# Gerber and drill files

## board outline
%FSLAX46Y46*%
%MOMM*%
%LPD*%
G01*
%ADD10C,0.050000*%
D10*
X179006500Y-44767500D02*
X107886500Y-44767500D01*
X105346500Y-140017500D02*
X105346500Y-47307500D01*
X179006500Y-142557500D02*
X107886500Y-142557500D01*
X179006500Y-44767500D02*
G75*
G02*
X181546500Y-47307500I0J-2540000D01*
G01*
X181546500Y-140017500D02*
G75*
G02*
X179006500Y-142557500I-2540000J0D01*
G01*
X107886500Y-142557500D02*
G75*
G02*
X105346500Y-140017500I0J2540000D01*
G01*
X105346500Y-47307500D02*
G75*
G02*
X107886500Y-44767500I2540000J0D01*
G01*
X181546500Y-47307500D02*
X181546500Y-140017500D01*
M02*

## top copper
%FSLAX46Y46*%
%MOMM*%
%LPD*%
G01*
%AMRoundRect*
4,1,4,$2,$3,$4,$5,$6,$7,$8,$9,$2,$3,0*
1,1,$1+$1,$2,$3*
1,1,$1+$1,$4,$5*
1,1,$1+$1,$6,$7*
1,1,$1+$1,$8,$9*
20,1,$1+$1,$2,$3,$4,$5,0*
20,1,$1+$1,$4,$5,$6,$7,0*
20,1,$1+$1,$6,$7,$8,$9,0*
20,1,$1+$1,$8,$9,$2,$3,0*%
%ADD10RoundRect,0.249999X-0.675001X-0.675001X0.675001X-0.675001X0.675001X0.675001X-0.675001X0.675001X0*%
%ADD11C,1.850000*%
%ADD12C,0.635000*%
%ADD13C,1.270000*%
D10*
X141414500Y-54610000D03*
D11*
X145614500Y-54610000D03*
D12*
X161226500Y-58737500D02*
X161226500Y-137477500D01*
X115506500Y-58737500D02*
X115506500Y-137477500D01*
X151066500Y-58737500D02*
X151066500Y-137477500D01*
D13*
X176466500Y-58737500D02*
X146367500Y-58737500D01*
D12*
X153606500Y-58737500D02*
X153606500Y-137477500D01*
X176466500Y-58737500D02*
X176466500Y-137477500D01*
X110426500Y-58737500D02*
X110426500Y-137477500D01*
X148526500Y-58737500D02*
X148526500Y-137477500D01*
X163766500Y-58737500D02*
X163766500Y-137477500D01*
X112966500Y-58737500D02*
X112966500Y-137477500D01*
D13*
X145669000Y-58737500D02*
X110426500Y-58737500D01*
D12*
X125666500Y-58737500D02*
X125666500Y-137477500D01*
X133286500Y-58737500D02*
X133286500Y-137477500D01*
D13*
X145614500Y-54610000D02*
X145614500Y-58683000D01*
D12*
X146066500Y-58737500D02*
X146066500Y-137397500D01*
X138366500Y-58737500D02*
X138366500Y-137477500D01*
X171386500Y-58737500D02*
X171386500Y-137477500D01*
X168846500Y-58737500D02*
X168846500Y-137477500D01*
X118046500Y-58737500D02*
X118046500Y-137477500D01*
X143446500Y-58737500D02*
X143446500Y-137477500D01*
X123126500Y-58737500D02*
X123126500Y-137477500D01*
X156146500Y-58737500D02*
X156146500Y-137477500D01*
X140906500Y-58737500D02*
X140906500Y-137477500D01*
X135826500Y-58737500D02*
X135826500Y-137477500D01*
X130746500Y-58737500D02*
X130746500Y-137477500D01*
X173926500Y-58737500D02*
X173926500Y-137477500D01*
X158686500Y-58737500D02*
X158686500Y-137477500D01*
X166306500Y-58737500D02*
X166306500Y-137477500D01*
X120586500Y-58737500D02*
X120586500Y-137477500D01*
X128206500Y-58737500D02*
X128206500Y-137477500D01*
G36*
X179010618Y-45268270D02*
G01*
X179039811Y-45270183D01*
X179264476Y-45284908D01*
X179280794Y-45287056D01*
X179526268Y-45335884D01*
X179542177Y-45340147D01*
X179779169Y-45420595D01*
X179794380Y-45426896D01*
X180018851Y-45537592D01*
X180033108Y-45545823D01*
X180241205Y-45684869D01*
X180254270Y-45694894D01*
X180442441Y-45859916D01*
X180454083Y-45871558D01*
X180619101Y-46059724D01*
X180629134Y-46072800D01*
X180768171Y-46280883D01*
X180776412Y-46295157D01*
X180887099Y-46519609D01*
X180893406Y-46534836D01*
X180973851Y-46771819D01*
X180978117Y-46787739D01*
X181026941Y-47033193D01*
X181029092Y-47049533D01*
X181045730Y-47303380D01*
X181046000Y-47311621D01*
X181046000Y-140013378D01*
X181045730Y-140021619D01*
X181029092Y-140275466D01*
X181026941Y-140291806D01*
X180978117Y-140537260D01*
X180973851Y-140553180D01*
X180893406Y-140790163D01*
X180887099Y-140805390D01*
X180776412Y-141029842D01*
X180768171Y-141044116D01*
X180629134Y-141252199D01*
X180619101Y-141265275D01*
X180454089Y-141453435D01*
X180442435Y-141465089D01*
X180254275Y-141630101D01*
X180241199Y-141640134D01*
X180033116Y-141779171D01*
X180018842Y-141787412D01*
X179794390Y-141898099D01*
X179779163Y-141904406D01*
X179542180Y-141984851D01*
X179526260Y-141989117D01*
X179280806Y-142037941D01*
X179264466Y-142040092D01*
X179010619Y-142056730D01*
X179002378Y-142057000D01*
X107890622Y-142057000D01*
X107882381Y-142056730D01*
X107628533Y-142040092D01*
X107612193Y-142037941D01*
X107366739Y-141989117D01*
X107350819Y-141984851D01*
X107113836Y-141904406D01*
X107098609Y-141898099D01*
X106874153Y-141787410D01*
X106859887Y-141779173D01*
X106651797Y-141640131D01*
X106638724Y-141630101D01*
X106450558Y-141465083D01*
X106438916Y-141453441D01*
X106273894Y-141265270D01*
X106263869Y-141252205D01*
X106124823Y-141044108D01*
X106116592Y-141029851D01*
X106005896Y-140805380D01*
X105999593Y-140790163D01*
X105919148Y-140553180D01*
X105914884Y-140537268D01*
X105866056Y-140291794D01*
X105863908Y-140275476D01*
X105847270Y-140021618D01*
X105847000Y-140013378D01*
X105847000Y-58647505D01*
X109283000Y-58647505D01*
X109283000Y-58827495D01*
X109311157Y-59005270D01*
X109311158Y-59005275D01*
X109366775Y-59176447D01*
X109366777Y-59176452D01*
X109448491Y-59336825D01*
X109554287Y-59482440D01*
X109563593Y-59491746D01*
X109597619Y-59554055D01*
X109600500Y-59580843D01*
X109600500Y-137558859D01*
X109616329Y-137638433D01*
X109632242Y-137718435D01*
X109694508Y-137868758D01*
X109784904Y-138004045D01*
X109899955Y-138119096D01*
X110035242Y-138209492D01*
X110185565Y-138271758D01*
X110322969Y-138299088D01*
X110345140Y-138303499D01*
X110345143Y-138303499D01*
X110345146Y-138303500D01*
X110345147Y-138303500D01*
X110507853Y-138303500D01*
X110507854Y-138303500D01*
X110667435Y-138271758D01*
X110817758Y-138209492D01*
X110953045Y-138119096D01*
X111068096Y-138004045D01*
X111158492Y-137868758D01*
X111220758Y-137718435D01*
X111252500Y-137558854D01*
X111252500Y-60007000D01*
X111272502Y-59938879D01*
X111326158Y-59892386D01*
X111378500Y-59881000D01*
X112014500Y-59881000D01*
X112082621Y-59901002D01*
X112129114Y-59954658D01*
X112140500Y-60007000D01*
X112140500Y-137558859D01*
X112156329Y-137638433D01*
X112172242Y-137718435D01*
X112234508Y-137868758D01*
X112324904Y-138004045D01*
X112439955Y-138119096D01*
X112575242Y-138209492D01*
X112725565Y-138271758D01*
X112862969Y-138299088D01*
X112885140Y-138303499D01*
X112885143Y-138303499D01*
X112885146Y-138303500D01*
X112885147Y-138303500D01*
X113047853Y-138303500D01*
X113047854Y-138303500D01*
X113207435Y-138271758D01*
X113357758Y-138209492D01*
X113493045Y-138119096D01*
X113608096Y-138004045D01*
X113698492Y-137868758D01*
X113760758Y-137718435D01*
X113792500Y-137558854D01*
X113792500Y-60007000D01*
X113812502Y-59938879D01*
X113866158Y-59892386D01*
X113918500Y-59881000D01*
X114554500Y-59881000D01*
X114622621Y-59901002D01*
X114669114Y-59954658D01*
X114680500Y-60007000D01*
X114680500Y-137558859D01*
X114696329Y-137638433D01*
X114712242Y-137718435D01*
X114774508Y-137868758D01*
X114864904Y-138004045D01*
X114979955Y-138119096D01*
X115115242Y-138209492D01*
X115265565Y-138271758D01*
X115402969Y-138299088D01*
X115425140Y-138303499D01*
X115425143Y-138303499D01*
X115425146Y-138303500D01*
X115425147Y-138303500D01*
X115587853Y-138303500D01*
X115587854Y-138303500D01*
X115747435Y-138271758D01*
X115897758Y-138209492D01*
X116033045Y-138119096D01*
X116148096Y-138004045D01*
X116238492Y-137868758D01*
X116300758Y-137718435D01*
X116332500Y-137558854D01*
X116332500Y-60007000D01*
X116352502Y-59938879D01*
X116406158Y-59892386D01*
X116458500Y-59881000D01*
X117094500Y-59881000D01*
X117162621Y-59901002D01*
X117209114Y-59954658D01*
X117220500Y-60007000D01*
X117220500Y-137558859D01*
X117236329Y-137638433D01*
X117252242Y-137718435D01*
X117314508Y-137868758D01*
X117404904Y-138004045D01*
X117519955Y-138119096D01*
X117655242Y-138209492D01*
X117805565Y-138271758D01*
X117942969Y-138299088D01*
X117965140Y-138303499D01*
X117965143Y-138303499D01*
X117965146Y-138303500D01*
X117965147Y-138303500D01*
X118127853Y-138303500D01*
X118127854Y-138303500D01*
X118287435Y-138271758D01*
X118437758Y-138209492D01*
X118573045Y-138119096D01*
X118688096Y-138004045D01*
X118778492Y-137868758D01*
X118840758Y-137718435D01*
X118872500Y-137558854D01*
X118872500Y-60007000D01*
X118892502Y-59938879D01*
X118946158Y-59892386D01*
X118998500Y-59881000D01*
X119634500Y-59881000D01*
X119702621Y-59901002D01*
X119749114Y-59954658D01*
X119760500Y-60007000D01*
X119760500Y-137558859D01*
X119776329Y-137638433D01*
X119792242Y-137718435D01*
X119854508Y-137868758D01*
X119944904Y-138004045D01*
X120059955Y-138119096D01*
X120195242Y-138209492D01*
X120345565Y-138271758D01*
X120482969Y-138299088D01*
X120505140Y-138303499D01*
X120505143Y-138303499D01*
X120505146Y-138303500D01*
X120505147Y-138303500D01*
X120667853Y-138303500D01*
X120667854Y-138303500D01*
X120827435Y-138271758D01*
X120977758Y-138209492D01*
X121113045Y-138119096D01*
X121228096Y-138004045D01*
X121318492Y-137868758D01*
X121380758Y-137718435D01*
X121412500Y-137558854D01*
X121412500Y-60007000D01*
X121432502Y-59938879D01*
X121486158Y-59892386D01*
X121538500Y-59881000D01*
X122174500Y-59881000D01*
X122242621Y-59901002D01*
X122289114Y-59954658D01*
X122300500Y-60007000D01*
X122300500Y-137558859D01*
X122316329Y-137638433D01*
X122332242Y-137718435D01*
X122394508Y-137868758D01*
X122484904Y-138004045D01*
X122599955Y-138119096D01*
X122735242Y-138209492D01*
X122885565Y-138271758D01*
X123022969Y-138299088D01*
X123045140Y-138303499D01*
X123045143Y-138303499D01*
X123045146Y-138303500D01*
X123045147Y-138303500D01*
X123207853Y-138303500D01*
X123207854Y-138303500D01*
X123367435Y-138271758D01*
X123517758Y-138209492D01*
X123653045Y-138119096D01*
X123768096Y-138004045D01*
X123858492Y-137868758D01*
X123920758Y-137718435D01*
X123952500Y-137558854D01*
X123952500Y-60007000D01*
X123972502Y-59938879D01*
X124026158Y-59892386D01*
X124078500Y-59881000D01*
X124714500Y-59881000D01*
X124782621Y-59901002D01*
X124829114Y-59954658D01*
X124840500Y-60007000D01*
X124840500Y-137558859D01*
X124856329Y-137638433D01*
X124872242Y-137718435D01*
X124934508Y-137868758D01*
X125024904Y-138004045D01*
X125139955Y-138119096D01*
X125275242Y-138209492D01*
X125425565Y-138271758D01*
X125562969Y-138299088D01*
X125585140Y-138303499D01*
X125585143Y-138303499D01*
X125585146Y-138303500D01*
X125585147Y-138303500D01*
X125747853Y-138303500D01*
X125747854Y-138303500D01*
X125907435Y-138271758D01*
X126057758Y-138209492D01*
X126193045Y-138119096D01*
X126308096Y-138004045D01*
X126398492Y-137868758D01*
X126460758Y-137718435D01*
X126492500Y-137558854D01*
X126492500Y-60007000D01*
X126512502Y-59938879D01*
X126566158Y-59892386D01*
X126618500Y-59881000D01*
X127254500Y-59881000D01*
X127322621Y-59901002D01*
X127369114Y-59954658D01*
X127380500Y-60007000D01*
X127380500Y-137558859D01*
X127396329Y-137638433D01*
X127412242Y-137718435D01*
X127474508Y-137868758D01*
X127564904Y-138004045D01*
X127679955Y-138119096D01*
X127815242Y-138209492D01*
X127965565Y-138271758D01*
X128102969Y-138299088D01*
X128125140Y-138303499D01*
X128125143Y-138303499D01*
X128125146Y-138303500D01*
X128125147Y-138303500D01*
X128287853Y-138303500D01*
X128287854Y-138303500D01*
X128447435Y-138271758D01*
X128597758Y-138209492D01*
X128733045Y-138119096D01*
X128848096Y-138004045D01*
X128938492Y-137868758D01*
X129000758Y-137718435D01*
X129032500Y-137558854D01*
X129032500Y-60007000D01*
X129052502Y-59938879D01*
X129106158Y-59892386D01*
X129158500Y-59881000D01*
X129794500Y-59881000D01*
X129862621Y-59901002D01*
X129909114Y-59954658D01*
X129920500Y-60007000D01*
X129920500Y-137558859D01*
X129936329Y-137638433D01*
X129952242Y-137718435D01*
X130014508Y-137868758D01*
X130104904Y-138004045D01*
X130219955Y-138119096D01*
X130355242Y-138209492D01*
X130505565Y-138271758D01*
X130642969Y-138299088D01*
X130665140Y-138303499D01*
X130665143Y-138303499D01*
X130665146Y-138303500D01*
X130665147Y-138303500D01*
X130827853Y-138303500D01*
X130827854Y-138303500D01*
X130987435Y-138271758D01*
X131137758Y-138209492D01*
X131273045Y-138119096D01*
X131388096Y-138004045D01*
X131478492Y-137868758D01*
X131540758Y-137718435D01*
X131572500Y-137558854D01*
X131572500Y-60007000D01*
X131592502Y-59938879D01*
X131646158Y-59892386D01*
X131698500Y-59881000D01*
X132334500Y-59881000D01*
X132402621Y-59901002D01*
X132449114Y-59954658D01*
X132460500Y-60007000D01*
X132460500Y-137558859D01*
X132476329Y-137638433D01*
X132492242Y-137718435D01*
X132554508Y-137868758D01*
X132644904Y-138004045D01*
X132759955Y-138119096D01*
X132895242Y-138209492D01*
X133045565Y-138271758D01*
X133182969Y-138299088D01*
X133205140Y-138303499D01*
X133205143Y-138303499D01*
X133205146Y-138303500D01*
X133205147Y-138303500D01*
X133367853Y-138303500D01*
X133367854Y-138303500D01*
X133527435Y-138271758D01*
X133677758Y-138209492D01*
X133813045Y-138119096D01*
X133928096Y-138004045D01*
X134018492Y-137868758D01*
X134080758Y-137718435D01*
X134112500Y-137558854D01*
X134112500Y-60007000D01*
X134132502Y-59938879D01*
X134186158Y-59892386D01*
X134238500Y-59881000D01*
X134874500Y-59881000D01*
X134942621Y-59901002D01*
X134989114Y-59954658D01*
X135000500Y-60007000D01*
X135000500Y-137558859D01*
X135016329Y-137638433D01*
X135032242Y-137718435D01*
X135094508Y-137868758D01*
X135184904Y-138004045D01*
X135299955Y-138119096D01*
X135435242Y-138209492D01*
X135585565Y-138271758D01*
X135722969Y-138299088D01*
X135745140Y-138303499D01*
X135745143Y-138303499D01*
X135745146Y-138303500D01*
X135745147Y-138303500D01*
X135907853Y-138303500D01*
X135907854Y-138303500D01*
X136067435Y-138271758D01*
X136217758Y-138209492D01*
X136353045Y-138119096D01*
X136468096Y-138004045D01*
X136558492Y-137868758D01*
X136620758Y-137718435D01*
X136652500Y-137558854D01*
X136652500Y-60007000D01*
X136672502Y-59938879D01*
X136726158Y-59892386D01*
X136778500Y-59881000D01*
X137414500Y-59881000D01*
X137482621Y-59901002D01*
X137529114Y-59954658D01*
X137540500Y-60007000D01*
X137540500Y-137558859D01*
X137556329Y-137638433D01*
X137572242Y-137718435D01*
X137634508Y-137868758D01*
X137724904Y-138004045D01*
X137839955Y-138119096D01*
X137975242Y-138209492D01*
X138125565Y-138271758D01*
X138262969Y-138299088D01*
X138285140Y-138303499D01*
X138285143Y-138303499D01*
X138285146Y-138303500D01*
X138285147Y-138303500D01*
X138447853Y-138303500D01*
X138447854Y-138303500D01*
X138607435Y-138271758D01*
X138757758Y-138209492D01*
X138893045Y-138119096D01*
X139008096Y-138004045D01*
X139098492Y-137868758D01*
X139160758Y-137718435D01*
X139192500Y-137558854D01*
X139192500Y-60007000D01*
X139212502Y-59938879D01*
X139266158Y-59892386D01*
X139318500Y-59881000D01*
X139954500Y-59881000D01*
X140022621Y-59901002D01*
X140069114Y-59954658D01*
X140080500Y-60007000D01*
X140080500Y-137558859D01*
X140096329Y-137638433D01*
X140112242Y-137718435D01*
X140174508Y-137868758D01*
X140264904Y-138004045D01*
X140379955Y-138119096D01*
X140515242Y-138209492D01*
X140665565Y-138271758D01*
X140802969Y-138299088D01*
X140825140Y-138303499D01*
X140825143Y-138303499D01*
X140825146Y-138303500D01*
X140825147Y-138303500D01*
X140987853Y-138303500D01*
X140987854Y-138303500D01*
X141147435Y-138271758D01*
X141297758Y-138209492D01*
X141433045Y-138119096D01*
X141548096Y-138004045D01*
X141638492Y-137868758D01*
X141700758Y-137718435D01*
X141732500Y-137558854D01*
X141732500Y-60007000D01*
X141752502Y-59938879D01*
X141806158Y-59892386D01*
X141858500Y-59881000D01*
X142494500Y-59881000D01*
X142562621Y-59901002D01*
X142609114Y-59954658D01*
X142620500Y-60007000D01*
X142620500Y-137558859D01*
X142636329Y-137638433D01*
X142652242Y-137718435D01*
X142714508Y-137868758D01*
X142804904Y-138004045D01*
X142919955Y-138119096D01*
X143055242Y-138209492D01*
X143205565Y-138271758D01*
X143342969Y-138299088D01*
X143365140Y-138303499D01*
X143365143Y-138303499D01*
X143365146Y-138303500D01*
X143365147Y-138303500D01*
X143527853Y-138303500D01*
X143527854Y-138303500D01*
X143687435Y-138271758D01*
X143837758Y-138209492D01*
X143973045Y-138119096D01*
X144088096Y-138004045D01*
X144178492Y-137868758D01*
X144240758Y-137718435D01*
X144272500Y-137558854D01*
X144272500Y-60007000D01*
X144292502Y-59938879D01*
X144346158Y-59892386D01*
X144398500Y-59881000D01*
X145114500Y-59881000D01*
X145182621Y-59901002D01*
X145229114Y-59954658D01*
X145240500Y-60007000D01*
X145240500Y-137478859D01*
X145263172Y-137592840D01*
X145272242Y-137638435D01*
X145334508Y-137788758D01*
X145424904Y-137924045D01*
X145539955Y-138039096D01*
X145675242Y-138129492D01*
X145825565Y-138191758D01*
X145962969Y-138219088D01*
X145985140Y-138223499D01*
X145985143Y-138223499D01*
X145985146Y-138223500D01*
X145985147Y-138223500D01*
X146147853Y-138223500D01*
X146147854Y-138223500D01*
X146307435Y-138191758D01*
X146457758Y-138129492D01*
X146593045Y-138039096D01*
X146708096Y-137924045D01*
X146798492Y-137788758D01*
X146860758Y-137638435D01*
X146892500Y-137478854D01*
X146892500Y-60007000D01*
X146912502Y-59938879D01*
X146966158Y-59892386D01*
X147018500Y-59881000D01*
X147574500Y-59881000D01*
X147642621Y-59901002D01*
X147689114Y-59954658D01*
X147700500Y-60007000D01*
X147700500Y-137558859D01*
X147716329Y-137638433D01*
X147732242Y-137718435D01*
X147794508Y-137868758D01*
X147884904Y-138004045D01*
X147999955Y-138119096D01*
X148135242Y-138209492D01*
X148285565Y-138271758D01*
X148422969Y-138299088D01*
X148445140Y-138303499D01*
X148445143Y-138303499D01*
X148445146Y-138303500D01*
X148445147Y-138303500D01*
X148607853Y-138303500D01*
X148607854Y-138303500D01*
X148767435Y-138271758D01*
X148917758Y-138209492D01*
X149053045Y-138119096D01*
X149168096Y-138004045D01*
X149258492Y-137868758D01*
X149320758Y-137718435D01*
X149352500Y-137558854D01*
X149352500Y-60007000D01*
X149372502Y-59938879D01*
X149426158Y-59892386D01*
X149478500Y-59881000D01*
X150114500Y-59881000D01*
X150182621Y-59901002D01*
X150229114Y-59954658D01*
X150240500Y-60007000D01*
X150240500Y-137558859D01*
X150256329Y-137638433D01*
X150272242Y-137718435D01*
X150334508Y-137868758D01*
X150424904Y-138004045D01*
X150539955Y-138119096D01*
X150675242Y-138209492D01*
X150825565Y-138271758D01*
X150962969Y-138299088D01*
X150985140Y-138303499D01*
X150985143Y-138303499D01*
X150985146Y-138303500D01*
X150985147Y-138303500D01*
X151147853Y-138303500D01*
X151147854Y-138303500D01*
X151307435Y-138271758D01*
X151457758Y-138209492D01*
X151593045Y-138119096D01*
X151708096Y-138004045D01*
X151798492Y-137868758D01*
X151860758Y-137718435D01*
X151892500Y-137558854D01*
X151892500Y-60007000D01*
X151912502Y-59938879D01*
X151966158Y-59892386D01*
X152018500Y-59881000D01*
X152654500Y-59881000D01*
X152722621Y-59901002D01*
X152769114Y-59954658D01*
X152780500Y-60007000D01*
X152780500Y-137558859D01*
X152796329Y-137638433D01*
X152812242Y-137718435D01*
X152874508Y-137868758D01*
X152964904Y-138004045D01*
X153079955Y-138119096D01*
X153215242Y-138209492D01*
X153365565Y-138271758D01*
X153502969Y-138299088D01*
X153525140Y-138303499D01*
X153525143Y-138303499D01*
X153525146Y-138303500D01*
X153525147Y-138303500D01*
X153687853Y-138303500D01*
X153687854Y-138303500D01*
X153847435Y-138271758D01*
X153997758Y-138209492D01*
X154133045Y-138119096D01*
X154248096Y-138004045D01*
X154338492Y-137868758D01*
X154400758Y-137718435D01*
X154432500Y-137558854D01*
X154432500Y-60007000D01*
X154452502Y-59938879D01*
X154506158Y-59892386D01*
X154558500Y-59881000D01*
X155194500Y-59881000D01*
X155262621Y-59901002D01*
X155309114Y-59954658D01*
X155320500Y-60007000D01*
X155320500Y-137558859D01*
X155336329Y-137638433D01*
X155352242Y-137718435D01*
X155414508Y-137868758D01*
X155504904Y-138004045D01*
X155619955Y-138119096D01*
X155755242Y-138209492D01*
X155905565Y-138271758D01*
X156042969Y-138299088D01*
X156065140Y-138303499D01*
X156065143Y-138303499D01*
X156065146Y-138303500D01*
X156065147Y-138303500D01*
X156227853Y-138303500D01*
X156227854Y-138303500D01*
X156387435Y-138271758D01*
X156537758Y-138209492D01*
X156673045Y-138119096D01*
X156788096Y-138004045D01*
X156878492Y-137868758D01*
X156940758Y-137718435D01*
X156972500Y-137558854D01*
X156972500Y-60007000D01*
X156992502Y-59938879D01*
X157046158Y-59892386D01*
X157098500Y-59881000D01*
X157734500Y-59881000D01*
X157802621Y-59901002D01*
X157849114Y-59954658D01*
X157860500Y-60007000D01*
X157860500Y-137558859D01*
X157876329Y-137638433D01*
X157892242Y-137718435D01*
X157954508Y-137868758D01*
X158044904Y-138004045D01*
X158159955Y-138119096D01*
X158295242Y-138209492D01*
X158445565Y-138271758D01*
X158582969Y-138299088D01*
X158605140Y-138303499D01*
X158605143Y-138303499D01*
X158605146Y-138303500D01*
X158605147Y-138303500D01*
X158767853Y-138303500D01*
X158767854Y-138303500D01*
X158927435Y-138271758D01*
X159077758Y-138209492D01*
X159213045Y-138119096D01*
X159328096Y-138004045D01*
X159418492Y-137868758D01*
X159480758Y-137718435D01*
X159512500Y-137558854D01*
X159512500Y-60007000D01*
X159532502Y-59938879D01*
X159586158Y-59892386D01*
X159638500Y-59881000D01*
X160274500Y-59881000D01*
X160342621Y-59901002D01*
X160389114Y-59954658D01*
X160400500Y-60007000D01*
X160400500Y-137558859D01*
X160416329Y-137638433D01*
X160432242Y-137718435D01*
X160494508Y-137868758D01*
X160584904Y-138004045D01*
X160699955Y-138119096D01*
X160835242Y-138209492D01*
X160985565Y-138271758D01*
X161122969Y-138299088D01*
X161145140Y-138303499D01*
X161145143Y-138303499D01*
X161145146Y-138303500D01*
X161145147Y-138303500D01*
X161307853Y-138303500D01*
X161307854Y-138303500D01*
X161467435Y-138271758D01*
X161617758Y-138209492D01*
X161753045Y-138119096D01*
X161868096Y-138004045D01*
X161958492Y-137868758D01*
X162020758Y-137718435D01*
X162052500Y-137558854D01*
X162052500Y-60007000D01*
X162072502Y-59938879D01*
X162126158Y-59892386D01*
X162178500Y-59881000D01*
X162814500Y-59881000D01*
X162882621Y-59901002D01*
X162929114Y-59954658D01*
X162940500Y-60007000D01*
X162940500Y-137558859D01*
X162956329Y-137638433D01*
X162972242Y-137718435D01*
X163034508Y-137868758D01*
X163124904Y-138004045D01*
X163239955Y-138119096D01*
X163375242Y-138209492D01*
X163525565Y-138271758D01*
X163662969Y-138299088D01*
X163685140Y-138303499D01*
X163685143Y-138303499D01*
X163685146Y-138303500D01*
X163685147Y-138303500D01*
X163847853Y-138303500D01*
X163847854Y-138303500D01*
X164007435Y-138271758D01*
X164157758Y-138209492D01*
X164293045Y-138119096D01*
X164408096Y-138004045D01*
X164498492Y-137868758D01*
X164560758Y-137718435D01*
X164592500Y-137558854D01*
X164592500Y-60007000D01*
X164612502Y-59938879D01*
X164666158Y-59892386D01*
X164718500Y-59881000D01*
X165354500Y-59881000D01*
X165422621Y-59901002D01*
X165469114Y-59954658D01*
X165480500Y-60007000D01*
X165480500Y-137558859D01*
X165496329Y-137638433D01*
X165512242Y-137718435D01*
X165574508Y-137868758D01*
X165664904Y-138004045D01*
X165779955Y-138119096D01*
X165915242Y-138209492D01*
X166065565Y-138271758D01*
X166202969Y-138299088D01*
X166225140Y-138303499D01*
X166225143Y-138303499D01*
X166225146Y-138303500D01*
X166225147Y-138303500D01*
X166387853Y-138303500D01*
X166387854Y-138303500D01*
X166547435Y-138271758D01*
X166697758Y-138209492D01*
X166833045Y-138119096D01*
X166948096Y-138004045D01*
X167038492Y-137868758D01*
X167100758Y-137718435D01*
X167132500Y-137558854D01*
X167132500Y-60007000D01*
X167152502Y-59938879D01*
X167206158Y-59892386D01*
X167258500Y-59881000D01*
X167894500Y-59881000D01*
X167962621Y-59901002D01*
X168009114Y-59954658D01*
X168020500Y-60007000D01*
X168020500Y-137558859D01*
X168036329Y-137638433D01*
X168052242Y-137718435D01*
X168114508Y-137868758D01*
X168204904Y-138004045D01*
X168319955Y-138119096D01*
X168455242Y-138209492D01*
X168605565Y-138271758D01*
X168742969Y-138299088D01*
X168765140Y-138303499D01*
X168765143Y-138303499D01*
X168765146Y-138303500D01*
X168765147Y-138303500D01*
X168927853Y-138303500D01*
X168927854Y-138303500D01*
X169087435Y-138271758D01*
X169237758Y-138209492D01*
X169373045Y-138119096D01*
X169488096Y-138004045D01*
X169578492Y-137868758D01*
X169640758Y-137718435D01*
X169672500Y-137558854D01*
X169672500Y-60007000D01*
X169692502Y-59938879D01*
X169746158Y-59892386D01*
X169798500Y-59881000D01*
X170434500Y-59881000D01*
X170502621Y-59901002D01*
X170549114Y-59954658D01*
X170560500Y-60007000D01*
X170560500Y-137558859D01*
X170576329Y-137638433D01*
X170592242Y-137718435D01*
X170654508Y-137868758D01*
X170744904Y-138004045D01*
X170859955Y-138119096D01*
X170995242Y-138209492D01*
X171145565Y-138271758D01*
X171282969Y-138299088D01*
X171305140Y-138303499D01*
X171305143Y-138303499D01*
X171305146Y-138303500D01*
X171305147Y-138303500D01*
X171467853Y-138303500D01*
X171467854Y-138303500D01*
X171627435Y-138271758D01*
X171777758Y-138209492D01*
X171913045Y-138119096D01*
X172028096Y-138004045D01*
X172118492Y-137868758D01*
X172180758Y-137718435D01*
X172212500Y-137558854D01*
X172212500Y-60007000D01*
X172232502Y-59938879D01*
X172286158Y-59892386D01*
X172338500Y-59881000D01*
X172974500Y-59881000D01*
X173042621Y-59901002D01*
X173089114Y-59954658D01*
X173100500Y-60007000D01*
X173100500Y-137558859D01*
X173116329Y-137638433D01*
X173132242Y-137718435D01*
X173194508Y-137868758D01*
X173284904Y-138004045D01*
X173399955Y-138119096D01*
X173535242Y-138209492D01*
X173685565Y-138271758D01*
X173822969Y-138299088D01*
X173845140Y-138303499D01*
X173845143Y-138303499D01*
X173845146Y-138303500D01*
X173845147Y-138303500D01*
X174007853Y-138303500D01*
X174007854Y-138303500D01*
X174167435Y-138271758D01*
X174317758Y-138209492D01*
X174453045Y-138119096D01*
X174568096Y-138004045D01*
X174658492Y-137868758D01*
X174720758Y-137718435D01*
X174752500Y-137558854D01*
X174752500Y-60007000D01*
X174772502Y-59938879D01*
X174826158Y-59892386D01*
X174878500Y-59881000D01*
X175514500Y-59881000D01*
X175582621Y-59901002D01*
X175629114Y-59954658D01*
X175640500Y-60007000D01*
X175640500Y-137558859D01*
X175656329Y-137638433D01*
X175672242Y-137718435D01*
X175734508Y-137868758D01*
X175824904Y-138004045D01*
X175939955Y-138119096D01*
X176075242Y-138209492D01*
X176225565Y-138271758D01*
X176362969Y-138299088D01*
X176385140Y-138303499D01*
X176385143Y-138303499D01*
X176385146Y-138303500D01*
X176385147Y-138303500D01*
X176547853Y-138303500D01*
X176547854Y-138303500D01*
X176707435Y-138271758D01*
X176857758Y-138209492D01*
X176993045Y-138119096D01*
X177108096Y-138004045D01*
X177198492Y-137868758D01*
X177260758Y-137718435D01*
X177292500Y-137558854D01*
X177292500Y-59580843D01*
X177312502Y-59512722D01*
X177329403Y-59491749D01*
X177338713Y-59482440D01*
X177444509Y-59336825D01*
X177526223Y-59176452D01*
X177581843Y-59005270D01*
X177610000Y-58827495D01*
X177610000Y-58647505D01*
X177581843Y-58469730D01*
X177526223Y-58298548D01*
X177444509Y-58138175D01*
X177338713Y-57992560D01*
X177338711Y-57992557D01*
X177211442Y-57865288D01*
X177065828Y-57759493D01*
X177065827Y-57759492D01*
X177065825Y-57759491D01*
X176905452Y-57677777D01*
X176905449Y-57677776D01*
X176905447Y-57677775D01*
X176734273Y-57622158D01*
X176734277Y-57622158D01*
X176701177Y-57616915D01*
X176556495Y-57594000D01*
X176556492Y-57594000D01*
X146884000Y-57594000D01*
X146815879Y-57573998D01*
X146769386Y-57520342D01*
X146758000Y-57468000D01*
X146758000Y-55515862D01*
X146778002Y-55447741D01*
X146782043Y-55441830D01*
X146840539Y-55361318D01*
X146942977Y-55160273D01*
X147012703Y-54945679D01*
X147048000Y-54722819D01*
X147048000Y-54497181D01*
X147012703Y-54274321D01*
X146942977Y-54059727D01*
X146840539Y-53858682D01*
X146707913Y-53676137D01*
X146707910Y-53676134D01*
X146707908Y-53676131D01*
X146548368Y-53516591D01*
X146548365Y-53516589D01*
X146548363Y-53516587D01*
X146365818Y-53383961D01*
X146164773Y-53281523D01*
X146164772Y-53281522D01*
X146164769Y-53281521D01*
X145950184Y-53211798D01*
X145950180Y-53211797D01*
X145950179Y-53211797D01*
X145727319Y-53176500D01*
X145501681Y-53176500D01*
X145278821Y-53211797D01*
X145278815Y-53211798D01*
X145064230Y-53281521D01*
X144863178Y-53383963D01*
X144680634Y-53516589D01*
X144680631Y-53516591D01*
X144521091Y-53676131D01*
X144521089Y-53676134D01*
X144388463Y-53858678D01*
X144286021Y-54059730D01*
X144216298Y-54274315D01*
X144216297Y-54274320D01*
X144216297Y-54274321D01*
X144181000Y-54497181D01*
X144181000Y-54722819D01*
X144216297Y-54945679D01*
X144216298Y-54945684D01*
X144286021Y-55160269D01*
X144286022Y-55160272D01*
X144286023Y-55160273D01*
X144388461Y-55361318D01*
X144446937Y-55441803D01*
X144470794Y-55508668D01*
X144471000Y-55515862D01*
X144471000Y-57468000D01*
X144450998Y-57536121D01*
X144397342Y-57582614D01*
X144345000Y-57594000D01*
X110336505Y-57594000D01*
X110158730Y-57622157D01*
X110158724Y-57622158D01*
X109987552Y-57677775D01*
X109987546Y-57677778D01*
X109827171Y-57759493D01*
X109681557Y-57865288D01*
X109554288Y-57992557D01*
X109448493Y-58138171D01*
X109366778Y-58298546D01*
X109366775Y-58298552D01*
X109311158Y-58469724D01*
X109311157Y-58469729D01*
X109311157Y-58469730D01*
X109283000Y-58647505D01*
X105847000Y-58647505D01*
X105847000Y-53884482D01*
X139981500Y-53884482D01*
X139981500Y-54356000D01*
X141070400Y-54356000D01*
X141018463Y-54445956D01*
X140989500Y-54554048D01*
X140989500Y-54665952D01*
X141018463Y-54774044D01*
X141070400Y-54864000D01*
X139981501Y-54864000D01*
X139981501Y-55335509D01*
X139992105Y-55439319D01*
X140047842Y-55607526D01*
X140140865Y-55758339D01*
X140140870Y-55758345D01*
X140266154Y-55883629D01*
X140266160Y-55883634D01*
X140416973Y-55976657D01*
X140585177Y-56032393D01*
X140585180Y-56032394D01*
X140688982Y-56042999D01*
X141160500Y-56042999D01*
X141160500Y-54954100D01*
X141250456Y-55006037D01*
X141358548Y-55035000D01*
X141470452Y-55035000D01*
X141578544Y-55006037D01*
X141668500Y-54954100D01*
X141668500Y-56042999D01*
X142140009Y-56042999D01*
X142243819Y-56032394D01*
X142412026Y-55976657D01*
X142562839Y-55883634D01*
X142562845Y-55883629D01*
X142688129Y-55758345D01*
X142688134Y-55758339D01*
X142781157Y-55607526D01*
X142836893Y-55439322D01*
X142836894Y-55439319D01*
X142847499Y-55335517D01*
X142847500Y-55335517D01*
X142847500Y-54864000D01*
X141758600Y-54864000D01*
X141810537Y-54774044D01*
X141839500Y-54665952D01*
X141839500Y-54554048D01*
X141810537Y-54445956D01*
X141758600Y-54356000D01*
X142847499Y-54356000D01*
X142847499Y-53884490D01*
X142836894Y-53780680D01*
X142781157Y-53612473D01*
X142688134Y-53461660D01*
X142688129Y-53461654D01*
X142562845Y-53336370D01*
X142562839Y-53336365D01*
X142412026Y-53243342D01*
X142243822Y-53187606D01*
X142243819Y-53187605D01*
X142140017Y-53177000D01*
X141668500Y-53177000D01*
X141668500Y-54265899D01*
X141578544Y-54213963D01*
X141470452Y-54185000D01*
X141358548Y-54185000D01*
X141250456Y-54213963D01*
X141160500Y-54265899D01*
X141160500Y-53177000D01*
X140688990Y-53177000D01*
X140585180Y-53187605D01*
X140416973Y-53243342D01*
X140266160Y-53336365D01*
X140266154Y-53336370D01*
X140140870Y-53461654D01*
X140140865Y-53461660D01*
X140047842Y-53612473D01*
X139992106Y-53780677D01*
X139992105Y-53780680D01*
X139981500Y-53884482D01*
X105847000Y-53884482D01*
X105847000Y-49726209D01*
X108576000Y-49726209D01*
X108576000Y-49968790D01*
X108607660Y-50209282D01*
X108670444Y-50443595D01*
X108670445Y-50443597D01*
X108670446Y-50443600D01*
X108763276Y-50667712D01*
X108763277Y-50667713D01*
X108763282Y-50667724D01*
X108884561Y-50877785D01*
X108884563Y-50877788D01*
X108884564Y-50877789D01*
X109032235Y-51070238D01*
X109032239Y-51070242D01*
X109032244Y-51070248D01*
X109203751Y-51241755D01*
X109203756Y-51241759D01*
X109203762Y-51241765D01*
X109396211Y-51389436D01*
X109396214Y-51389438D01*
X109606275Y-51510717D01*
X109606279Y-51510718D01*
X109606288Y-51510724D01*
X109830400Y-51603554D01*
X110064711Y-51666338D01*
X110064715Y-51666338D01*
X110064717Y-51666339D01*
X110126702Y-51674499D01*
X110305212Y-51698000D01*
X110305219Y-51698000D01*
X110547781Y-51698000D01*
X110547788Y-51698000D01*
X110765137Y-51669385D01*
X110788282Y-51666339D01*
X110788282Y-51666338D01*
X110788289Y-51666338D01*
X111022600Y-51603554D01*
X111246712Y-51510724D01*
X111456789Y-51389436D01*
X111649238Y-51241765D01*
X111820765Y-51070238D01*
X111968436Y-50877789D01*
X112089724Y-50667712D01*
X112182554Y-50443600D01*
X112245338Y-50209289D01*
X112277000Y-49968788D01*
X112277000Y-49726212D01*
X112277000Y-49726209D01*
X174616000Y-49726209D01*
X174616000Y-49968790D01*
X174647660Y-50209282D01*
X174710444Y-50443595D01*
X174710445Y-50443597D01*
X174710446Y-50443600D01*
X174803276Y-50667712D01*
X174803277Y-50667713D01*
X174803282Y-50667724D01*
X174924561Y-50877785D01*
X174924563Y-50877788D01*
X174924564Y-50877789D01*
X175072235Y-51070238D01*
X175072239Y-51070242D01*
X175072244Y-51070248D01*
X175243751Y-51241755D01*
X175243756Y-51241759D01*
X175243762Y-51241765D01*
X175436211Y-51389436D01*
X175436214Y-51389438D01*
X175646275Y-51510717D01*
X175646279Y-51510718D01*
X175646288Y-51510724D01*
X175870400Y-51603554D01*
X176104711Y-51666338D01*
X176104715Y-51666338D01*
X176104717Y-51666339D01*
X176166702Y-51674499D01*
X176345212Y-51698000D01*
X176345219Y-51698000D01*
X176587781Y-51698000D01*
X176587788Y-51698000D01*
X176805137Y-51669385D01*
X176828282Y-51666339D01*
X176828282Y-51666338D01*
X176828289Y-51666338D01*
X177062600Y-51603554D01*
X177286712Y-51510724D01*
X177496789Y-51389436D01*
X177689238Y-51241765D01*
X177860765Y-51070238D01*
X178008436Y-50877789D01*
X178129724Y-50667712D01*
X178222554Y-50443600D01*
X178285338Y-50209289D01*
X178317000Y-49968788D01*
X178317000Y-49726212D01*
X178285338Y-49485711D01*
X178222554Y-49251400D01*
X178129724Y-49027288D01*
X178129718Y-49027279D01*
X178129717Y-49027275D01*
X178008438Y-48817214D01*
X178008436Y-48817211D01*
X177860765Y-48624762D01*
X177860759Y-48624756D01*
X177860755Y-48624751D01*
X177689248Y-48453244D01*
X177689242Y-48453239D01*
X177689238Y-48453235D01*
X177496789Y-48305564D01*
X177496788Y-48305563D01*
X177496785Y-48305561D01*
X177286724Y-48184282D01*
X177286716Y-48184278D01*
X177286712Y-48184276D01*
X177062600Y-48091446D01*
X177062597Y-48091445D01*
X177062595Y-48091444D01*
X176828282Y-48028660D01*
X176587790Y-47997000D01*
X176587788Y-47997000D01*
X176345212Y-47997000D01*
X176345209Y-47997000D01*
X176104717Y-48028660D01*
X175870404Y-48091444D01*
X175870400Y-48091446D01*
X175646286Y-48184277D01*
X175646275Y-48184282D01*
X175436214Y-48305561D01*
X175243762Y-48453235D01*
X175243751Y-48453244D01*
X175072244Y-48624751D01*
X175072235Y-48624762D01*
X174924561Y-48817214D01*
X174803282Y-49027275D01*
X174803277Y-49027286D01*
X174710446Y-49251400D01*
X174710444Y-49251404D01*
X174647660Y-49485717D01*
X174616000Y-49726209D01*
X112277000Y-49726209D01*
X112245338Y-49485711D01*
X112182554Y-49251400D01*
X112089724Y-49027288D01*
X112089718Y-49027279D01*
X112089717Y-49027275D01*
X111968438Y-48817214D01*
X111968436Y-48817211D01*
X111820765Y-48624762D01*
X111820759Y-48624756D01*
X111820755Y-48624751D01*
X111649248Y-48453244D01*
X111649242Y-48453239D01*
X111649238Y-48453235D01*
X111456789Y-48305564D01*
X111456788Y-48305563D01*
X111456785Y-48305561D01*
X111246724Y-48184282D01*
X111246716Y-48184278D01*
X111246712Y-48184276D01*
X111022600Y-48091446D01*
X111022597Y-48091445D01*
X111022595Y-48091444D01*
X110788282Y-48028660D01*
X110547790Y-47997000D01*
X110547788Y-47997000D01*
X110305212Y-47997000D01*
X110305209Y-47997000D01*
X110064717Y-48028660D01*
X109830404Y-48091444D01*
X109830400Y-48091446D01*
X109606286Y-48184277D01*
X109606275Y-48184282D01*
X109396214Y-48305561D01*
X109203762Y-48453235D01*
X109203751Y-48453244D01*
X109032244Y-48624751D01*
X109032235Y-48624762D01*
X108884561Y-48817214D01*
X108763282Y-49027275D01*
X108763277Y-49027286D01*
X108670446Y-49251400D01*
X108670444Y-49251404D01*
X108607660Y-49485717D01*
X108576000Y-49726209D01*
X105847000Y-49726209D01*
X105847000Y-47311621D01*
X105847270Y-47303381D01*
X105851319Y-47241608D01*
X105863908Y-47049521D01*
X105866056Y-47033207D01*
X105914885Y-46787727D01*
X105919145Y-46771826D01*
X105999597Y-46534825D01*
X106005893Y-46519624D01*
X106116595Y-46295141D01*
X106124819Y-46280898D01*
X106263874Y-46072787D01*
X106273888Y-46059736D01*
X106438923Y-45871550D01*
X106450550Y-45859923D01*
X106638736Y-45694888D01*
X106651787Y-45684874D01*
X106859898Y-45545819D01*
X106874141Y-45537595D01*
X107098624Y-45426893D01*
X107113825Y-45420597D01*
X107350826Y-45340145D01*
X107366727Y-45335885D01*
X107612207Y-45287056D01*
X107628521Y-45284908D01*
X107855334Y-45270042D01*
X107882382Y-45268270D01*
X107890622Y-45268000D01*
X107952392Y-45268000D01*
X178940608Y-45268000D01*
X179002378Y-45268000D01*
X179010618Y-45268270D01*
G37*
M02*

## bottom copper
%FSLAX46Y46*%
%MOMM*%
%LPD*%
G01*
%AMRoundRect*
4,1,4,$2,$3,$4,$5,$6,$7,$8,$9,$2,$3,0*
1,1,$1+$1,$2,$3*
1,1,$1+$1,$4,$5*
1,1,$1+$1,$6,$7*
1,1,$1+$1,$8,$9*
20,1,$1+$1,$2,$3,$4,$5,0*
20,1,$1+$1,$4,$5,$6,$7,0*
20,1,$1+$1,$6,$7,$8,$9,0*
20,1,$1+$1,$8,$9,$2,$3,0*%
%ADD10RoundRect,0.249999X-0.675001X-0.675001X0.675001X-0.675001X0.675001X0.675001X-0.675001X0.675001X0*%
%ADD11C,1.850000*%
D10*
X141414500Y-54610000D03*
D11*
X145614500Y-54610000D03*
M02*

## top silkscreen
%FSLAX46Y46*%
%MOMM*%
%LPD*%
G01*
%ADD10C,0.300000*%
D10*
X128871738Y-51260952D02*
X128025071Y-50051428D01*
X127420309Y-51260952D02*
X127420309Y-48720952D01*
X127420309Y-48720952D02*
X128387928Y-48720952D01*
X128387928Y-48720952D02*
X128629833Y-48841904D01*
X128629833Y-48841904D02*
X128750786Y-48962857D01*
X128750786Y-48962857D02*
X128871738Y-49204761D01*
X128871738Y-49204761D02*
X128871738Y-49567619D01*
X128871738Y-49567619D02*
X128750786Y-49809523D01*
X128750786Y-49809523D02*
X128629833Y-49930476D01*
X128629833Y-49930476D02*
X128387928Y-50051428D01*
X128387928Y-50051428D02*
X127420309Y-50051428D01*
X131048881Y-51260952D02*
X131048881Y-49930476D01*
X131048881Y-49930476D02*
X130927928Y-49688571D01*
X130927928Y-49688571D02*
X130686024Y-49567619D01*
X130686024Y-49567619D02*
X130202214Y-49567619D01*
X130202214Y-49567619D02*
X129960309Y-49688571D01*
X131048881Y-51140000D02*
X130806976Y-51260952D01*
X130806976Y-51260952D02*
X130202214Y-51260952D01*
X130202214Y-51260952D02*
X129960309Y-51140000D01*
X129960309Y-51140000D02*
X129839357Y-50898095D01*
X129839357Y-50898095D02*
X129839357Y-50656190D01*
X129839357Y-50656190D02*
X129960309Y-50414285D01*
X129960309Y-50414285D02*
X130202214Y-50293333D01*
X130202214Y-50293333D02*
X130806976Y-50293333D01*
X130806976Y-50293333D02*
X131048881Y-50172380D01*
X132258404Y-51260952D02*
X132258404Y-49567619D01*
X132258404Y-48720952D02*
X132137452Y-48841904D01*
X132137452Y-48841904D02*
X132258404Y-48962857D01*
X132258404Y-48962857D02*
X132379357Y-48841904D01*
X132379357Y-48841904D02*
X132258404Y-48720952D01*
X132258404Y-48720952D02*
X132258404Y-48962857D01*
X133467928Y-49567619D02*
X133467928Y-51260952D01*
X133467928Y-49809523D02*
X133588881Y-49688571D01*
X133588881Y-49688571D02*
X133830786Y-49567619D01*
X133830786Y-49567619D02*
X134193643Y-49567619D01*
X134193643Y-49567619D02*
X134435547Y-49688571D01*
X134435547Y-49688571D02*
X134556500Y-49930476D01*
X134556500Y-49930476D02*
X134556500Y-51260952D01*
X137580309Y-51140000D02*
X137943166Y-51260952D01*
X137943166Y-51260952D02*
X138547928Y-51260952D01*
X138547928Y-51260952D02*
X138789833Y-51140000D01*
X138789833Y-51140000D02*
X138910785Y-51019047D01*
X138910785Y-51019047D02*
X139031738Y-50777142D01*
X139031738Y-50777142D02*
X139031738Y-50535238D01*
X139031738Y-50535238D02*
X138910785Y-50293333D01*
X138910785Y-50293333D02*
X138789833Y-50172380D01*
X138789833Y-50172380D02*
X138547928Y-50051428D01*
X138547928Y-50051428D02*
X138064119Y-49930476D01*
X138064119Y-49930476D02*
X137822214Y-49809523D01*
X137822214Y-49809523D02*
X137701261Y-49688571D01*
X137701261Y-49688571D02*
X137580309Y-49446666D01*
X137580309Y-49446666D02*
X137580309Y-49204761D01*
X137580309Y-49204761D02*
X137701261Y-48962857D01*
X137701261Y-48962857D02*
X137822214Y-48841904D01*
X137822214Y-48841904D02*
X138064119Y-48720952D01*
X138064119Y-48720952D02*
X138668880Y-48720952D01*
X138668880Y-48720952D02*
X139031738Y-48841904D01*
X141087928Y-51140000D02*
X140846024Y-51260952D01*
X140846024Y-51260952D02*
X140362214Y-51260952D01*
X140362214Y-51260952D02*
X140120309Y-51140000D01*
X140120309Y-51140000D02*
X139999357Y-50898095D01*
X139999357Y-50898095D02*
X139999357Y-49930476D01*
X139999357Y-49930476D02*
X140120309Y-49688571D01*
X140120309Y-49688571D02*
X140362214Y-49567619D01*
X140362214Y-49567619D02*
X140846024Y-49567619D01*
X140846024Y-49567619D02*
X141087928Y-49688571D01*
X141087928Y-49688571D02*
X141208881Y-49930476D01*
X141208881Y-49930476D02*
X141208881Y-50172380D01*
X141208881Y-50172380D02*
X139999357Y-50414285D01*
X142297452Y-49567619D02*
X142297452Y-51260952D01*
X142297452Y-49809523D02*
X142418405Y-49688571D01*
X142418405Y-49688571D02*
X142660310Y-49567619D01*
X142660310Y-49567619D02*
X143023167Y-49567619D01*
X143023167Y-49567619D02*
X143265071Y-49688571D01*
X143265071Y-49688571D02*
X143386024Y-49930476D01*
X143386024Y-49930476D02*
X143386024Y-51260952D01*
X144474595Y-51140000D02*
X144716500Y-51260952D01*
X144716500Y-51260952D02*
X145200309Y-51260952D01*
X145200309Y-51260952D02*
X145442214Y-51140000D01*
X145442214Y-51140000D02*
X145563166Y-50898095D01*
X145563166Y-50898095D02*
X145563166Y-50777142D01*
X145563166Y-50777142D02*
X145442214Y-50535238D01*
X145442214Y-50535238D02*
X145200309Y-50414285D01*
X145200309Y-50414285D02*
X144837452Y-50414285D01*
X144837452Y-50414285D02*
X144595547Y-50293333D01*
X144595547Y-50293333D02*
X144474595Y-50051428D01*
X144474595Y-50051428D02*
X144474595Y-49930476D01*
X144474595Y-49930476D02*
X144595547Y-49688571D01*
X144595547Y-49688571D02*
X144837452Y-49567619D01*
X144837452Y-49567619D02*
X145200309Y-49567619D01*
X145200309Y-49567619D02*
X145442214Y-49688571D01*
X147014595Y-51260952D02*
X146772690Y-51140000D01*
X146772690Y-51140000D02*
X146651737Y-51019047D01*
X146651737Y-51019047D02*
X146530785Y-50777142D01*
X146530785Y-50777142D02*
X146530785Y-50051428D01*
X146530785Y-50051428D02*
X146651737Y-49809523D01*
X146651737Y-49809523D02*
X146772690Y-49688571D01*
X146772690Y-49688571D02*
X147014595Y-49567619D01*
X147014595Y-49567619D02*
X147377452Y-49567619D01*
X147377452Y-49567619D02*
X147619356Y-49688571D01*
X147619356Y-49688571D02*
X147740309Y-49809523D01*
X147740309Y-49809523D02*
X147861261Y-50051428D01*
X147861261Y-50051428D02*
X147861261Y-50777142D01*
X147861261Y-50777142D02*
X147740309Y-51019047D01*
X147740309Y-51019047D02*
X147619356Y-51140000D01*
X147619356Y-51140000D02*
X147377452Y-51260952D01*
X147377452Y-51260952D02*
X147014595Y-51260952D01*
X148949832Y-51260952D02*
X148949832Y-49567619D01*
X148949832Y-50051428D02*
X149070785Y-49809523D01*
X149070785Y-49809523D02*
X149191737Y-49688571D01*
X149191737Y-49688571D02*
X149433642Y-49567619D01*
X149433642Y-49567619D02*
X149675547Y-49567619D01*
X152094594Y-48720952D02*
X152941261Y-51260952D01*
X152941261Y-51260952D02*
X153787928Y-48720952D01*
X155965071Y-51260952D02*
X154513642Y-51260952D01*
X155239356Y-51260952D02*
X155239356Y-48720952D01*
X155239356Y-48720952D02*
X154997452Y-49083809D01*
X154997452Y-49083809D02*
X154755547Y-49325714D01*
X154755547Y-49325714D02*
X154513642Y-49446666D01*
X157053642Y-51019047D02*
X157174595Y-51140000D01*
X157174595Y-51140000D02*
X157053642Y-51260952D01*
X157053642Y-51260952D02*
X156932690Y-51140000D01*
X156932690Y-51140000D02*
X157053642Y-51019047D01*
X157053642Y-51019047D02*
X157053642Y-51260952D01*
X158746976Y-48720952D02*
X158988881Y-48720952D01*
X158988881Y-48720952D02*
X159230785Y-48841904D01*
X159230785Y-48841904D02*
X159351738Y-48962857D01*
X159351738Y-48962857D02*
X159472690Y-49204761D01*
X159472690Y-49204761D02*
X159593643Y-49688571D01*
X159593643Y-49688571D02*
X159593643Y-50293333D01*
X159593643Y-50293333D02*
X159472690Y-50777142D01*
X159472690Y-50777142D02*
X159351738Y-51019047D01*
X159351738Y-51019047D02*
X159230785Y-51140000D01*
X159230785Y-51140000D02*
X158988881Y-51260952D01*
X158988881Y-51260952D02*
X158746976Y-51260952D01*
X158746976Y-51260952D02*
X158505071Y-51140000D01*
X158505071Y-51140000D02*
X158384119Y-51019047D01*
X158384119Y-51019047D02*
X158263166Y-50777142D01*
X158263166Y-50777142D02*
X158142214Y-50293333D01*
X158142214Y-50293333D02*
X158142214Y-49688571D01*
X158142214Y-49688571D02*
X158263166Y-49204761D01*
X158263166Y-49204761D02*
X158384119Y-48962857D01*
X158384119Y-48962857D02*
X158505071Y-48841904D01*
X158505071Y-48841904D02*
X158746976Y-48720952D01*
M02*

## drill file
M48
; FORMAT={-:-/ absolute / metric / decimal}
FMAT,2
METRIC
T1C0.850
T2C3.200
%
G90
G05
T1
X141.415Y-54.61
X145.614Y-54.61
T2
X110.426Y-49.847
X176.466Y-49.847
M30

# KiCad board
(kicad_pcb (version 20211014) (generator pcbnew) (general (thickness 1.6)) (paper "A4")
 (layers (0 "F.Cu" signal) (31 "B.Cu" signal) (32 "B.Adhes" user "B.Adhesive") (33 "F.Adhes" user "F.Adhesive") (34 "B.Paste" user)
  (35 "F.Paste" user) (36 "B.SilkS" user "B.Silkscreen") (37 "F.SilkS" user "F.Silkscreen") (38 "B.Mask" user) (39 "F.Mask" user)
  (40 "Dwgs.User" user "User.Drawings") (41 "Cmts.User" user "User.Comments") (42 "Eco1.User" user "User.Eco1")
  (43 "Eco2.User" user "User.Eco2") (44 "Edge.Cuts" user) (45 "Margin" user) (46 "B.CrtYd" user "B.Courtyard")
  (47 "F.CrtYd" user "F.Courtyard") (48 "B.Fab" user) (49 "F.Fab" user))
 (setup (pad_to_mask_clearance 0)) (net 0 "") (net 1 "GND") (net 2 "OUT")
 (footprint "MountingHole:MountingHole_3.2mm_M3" (layer "F.Cu") (at 110.4265 49.8475 180)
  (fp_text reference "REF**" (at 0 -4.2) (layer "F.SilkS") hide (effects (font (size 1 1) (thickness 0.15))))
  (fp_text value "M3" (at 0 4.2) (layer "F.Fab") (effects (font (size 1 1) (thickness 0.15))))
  (pad "" np_thru_hole circle locked (at 0 0 180) (size 3.2 3.2) (drill 3.2) (layers *.Cu *.Mask)))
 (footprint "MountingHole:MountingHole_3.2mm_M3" (layer "F.Cu") (at 176.4665 49.8475 180)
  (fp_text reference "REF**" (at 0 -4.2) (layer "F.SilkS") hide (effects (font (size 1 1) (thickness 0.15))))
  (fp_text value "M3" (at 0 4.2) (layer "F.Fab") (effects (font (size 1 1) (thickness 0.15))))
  (pad "" np_thru_hole circle locked (at 0 0 180) (size 3.2 3.2) (drill 3.2) (layers *.Cu *.Mask)))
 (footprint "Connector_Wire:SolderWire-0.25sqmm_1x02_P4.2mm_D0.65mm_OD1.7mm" (layer "B.Cu") (at 141.4145 54.61)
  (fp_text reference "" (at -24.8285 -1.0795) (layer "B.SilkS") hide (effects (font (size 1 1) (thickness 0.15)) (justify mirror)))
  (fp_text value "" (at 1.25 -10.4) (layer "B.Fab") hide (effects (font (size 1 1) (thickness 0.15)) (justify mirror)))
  (pad "1" thru_hole roundrect locked (at 0 0) (size 1.85 1.85) (drill 0.85) (layers *.Cu *.Mask) (roundrect_rratio 0.1351345946)
   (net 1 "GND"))
  (pad "2" thru_hole circle locked (at 4.2 0) (size 1.85 1.85) (drill 0.85) (layers *.Cu *.Mask) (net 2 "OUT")))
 (gr_line (start 179.0065 44.7675) (end 107.8865 44.7675) (layer "Edge.Cuts") (width 0.05))
 (gr_line (start 105.3465 140.0175) (end 105.3465 47.3075) (layer "Edge.Cuts") (width 0.05))
 (gr_line (start 179.0065 142.5575) (end 107.8865 142.5575) (layer "Edge.Cuts") (width 0.05))
 (gr_arc (start 179.0065 44.7675) (mid 180.802551 45.511449) (end 181.5465 47.3075) (layer "Edge.Cuts") (width 0.05))
 (gr_arc (start 181.5465 140.0175) (mid 180.802551 141.813551) (end 179.0065 142.5575) (layer "Edge.Cuts") (width 0.05))
 (gr_arc (start 107.8865 142.5575) (mid 106.090449 141.813551) (end 105.3465 140.0175) (layer "Edge.Cuts") (width 0.05))
 (gr_arc (start 105.3465 47.3075) (mid 106.090449 45.511449) (end 107.8865 44.7675) (layer "Edge.Cuts") (width 0.05))
 (gr_line (start 181.5465 47.3075) (end 181.5465 140.0175) (layer "Edge.Cuts") (width 0.05))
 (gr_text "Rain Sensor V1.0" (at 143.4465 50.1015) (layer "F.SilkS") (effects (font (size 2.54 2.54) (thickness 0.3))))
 (segment (start 161.2265 58.7375) (end 161.2265 137.4775) (width 0.635) (layer "F.Cu") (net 2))
 (segment (start 115.5065 58.7375) (end 115.5065 137.4775) (width 0.635) (layer "F.Cu") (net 2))
 (segment (start 151.0665 58.7375) (end 151.0665 137.4775) (width 0.635) (layer "F.Cu") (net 2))
 (segment (start 176.4665 58.7375) (end 146.3675 58.7375) (width 1.27) (layer "F.Cu") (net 2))
 (segment (start 153.6065 58.7375) (end 153.6065 137.4775) (width 0.635) (layer "F.Cu") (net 2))
 (segment (start 176.4665 58.7375) (end 176.4665 137.4775) (width 0.635) (layer "F.Cu") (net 2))
 (segment (start 110.4265 58.7375) (end 110.4265 137.4775) (width 0.635) (layer "F.Cu") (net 2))
 (segment (start 148.5265 58.7375) (end 148.5265 137.4775) (width 0.635) (layer "F.Cu") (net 2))
 (segment (start 163.7665 58.7375) (end 163.7665 137.4775) (width 0.635) (layer "F.Cu") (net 2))
 (segment (start 112.9665 58.7375) (end 112.9665 137.4775) (width 0.635) (layer "F.Cu") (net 2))
 (segment (start 145.669 58.7375) (end 110.4265 58.7375) (width 1.27) (layer "F.Cu") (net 2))
 (segment (start 125.6665 58.7375) (end 125.6665 137.4775) (width 0.635) (layer "F.Cu") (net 2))
 (segment (start 133.2865 58.7375) (end 133.2865 137.4775) (width 0.635) (layer "F.Cu") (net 2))
 (segment (start 145.6145 54.61) (end 145.6145 58.683) (width 1.27) (layer "F.Cu") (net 2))
 (segment (start 146.0665 58.7375) (end 146.0665 137.3975) (width 0.635) (layer "F.Cu") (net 2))
 (segment (start 138.3665 58.7375) (end 138.3665 137.4775) (width 0.635) (layer "F.Cu") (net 2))
 (segment (start 171.3865 58.7375) (end 171.3865 137.4775) (width 0.635) (layer "F.Cu") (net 2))
 (segment (start 168.8465 58.7375) (end 168.8465 137.4775) (width 0.635) (layer "F.Cu") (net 2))
 (segment (start 118.0465 58.7375) (end 118.0465 137.4775) (width 0.635) (layer "F.Cu") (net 2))
 (segment (start 143.4465 58.7375) (end 143.4465 137.4775) (width 0.635) (layer "F.Cu") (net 2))
 (segment (start 123.1265 58.7375) (end 123.1265 137.4775) (width 0.635) (layer "F.Cu") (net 2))
 (segment (start 156.1465 58.7375) (end 156.1465 137.4775) (width 0.635) (layer "F.Cu") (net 2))
 (segment (start 140.9065 58.7375) (end 140.9065 137.4775) (width 0.635) (layer "F.Cu") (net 2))
 (segment (start 135.8265 58.7375) (end 135.8265 137.4775) (width 0.635) (layer "F.Cu") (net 2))
 (segment (start 130.7465 58.7375) (end 130.7465 137.4775) (width 0.635) (layer "F.Cu") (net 2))
 (segment (start 173.9265 58.7375) (end 173.9265 137.4775) (width 0.635) (layer "F.Cu") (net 2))
 (segment (start 158.6865 58.7375) (end 158.6865 137.4775) (width 0.635) (layer "F.Cu") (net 2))
 (segment (start 166.3065 58.7375) (end 166.3065 137.4775) (width 0.635) (layer "F.Cu") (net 2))
 (segment (start 120.5865 58.7375) (end 120.5865 137.4775) (width 0.635) (layer "F.Cu") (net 2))
 (segment (start 128.2065 58.7375) (end 128.2065 137.4775) (width 0.635) (layer "F.Cu") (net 2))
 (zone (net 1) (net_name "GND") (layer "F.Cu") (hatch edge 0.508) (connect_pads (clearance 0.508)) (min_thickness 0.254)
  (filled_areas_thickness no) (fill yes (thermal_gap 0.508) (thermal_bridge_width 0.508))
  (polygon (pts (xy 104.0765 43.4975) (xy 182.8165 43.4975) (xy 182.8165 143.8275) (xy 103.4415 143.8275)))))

